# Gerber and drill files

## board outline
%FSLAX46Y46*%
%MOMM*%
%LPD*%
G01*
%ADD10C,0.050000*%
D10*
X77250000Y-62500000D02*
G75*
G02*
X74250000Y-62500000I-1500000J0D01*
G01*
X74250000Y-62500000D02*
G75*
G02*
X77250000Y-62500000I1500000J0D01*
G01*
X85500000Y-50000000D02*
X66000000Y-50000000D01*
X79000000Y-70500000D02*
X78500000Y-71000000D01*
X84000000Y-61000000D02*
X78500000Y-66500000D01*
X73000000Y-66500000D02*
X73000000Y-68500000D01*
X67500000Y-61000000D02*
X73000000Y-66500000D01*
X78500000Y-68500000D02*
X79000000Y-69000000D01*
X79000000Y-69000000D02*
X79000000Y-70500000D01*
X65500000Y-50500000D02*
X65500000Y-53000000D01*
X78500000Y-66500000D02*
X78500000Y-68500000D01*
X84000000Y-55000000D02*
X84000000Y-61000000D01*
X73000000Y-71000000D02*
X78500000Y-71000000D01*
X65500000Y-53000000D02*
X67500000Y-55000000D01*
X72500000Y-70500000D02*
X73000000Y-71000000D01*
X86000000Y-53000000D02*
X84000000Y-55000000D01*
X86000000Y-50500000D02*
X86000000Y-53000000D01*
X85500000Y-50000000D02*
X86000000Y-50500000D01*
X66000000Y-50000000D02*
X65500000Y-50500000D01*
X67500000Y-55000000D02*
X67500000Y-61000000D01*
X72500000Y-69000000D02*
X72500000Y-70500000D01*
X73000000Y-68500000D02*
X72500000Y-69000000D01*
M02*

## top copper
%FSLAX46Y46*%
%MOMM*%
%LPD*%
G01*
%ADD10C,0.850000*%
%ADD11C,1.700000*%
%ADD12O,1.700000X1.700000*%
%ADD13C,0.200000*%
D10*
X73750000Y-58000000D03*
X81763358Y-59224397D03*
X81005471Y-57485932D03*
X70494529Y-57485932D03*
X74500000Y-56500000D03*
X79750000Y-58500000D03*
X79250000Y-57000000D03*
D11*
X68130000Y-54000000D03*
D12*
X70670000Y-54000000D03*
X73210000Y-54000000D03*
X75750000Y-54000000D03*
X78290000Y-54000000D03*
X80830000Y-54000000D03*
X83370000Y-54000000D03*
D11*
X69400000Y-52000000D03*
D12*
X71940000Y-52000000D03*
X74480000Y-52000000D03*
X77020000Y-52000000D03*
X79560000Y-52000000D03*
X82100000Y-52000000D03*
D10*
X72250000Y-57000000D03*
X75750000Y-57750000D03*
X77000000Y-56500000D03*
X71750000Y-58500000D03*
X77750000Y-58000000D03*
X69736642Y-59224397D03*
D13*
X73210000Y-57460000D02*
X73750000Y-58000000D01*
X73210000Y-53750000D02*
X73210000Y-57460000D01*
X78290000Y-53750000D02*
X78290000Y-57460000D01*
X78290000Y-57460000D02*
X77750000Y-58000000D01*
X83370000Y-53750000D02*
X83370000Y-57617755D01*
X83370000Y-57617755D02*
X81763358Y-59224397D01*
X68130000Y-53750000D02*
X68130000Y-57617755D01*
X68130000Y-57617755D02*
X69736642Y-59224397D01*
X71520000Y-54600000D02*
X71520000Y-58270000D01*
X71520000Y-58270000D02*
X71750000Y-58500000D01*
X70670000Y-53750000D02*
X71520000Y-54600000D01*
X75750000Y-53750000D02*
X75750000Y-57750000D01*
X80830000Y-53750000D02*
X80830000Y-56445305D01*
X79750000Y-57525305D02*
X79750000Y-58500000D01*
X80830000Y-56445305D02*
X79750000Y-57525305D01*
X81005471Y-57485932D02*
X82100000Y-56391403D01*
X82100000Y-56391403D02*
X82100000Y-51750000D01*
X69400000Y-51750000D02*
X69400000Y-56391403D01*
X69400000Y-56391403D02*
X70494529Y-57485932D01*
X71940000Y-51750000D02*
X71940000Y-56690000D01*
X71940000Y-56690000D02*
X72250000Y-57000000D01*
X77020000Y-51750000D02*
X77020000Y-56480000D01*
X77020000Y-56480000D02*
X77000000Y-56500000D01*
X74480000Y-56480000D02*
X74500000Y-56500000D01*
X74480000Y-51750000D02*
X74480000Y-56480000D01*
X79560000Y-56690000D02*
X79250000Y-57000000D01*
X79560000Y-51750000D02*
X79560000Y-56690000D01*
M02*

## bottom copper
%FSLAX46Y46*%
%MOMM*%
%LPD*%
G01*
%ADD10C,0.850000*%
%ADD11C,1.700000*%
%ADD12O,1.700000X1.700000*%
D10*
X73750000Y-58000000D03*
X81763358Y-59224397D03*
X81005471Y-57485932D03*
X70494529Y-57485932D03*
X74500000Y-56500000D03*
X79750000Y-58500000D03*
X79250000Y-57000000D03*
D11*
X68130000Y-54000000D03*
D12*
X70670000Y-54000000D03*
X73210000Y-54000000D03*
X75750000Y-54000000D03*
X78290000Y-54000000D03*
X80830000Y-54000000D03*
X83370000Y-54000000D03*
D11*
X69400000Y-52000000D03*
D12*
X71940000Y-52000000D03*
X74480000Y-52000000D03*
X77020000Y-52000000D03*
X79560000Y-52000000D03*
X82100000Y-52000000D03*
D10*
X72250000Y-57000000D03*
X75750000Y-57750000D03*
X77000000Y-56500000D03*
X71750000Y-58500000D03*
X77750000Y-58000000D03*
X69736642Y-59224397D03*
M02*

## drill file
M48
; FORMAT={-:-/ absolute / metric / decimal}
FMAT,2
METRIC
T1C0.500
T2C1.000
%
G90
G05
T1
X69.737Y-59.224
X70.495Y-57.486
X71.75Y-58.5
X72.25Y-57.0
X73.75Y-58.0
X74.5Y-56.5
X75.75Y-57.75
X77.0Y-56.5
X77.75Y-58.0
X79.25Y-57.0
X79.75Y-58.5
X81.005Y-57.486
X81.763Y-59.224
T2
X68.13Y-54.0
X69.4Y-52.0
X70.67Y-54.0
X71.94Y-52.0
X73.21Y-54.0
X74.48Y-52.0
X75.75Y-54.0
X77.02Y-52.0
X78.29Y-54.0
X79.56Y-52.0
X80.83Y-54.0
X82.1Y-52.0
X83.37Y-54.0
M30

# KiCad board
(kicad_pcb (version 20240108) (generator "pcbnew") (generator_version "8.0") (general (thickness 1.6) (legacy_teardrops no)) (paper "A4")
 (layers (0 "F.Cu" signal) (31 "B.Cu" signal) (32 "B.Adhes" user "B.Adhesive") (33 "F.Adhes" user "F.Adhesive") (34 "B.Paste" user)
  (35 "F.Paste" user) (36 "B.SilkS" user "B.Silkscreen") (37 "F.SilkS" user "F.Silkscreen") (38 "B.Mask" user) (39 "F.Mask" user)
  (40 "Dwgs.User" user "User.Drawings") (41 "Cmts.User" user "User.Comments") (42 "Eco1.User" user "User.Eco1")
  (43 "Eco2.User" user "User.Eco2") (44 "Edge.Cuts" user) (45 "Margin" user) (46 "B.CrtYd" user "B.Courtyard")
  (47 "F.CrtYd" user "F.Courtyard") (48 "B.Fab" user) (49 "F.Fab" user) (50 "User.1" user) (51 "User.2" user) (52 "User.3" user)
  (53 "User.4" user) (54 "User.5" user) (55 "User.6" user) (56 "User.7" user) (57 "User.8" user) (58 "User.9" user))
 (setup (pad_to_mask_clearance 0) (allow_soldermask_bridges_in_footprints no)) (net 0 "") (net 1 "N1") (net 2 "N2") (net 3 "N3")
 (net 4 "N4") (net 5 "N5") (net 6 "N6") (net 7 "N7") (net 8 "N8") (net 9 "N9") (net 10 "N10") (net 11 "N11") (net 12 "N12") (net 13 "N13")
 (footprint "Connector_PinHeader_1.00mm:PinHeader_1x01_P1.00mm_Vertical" (layer "F.Cu") (at 73.75 58)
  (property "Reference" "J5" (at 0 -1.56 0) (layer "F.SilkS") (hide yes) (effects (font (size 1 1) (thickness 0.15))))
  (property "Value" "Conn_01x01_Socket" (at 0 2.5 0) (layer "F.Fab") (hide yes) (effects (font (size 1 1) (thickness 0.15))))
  (pad "1" thru_hole circle (at 0 0) (size 0.85 0.85) (drill 0.5) (layers "*.Cu" "*.Mask") (remove_unused_layers no) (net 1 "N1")))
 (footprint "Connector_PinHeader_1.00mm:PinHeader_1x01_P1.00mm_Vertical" (layer "F.Cu") (at 81.763358 59.224397)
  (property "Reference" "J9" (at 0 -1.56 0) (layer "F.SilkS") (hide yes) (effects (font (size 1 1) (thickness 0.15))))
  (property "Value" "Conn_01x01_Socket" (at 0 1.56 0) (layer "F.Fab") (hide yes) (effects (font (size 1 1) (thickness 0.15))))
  (pad "1" thru_hole circle (at 0 0) (size 0.85 0.85) (drill 0.5) (layers "*.Cu" "*.Mask") (remove_unused_layers no) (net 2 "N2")))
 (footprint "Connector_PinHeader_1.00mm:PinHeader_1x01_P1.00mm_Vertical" (layer "F.Cu") (at 81.005471 57.485932)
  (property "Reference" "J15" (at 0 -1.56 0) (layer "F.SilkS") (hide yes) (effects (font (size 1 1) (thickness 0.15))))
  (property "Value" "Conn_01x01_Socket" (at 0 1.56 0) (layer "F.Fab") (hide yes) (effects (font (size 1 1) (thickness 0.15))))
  (pad "1" thru_hole circle (at 0 0) (size 0.85 0.85) (drill 0.5) (layers "*.Cu" "*.Mask") (remove_unused_layers no) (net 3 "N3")))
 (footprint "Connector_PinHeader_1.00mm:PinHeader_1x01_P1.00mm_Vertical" (layer "F.Cu") (at 70.494529 57.485932)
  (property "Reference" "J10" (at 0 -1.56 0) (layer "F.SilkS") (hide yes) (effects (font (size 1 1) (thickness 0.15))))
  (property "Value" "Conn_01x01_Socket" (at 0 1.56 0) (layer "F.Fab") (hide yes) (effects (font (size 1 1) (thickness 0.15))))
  (pad "1" thru_hole circle (at 0 0) (size 0.85 0.85) (drill 0.5) (layers "*.Cu" "*.Mask") (remove_unused_layers no) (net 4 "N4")))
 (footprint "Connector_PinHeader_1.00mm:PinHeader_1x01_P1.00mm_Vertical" (layer "F.Cu") (at 74.5 56.5)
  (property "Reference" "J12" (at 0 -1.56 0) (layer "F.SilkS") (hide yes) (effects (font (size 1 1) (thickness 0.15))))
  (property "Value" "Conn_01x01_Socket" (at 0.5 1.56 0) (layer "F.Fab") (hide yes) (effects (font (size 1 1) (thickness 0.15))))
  (pad "1" thru_hole circle (at 0 0) (size 0.85 0.85) (drill 0.5) (layers "*.Cu" "*.Mask") (remove_unused_layers no) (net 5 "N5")))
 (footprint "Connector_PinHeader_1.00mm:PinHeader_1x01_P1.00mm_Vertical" (layer "F.Cu") (at 79.75 58.5)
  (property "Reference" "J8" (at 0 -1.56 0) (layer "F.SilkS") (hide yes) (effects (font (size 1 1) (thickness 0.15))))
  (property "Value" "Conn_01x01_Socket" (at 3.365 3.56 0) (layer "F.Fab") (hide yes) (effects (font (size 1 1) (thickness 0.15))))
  (pad "1" thru_hole circle (at 0 0) (size 0.85 0.85) (drill 0.5) (layers "*.Cu" "*.Mask") (remove_unused_layers no) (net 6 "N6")))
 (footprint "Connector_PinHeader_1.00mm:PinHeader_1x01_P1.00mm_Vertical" (layer "F.Cu") (at 79.25 57)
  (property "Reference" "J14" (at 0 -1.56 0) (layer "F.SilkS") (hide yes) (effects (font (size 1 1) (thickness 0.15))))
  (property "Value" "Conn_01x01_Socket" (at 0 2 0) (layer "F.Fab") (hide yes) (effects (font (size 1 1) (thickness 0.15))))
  (pad "1" thru_hole circle (at 0 0) (size 0.85 0.85) (drill 0.5) (layers "*.Cu" "*.Mask") (remove_unused_layers no) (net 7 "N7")))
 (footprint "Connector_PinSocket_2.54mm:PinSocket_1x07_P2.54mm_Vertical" (layer "F.Cu") (at 68.13 54 90)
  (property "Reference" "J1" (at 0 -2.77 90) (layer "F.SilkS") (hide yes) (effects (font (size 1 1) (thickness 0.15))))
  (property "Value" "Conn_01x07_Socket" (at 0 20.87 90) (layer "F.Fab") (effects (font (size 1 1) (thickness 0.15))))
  (pad "1" thru_hole circle (at 0 0 90) (size 1.7 1.7) (drill 1) (layers "*.Cu" "*.Mask") (remove_unused_layers no) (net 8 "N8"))
  (pad "2" thru_hole oval (at 0 2.54 90) (size 1.7 1.7) (drill 1) (layers "*.Cu" "*.Mask") (remove_unused_layers no) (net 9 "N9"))
  (pad "3" thru_hole oval (at 0 5.08 90) (size 1.7 1.7) (drill 1) (layers "*.Cu" "*.Mask") (remove_unused_layers no) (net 1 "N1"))
  (pad "4" thru_hole oval (at 0 7.62 90) (size 1.7 1.7) (drill 1) (layers "*.Cu" "*.Mask") (remove_unused_layers no) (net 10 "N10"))
  (pad "5" thru_hole oval (at 0 10.16 90) (size 1.7 1.7) (drill 1) (layers "*.Cu" "*.Mask") (remove_unused_layers no) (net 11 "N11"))
  (pad "6" thru_hole oval (at 0 12.7 90) (size 1.7 1.7) (drill 1) (layers "*.Cu" "*.Mask") (remove_unused_layers no) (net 6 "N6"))
  (pad "7" thru_hole oval (at 0 15.24 90) (size 1.7 1.7) (drill 1) (layers "*.Cu" "*.Mask") (remove_unused_layers no) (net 2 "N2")))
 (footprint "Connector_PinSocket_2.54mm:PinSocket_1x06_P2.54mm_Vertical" (layer "F.Cu") (at 69.4 52 90)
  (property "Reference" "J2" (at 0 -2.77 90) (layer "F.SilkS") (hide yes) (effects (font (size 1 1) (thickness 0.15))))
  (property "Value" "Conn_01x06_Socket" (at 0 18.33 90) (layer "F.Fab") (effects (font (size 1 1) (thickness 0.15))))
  (pad "1" thru_hole circle (at 0 0 90) (size 1.7 1.7) (drill 1) (layers "*.Cu" "*.Mask") (remove_unused_layers no) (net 4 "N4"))
  (pad "2" thru_hole oval (at 0 2.54 90) (size 1.7 1.7) (drill 1) (layers "*.Cu" "*.Mask") (remove_unused_layers no) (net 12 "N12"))
  (pad "3" thru_hole oval (at 0 5.08 90) (size 1.7 1.7) (drill 1) (layers "*.Cu" "*.Mask") (remove_unused_layers no) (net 5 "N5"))
  (pad "4" thru_hole oval (at 0 7.62 90) (size 1.7 1.7) (drill 1) (layers "*.Cu" "*.Mask") (remove_unused_layers no) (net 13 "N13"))
  (pad "5" thru_hole oval (at 0 10.16 90) (size 1.7 1.7) (drill 1) (layers "*.Cu" "*.Mask") (remove_unused_layers no) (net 7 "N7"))
  (pad "6" thru_hole oval (at 0 12.7 90) (size 1.7 1.7) (drill 1) (layers "*.Cu" "*.Mask") (remove_unused_layers no) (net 3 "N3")))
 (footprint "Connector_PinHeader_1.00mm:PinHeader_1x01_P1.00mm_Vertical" (layer "F.Cu") (at 72.25 57)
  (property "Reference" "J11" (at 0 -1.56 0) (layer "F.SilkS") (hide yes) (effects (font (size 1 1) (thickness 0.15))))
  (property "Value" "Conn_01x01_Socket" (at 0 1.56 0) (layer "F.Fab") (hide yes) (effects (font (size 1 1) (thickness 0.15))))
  (pad "1" thru_hole circle (at 0 0) (size 0.85 0.85) (drill 0.5) (layers "*.Cu" "*.Mask") (remove_unused_layers no) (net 12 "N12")))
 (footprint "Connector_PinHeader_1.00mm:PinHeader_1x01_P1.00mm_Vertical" (layer "F.Cu") (at 75.75 57.75)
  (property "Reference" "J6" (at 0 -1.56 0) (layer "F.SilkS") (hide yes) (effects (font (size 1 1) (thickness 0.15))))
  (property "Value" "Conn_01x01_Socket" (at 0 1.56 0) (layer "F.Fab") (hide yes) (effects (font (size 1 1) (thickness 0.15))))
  (pad "1" thru_hole circle (at 0 0) (size 0.85 0.85) (drill 0.5) (layers "*.Cu" "*.Mask") (remove_unused_layers no) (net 10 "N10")))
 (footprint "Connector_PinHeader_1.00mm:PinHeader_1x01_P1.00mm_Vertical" (layer "F.Cu") (at 77 56.5)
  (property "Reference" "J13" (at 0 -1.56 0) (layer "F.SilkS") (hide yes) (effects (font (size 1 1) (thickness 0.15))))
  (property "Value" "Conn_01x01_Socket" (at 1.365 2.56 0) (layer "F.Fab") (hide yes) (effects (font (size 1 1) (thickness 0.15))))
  (pad "1" thru_hole circle (at 0 0) (size 0.85 0.85) (drill 0.5) (layers "*.Cu" "*.Mask") (remove_unused_layers no) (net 13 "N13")))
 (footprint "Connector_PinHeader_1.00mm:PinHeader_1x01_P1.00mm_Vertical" (layer "F.Cu") (at 71.75 58.5)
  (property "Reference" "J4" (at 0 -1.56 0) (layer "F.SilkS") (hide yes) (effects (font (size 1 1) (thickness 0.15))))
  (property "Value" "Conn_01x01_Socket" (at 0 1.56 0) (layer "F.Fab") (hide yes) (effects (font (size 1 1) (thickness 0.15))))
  (pad "1" thru_hole circle (at 0 0) (size 0.85 0.85) (drill 0.5) (layers "*.Cu" "*.Mask") (remove_unused_layers no) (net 9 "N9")))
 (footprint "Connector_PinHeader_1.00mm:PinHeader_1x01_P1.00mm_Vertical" (layer "F.Cu") (at 77.75 58)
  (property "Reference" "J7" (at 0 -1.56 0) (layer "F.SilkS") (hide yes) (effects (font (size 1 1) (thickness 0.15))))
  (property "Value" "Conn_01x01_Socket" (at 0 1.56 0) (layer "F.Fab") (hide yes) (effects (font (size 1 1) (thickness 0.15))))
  (pad "1" thru_hole circle (at 0 0) (size 0.85 0.85) (drill 0.5) (layers "*.Cu" "*.Mask") (remove_unused_layers no) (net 11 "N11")))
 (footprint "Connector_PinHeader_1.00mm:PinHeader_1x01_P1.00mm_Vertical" (layer "F.Cu") (at 69.736642 59.224397)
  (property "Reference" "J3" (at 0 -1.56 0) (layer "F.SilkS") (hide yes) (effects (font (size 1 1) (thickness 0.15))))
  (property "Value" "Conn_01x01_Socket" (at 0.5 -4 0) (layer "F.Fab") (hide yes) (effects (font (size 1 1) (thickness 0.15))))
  (pad "1" thru_hole circle (at 0 0) (size 0.85 0.85) (drill 0.5) (layers "*.Cu" "*.Mask") (remove_unused_layers no) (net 8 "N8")))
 (gr_circle (center 75.75 62.5) (end 75.75 61) (stroke (width 0.05) (type default)) (fill none) (layer "Edge.Cuts"))
 (gr_line (start 85.5 50) (end 66 50) (stroke (width 0.05) (type default)) (layer "Edge.Cuts"))
 (gr_line (start 79 70.5) (end 78.5 71) (stroke (width 0.05) (type default)) (layer "Edge.Cuts"))
 (gr_line (start 84 61) (end 78.5 66.5) (stroke (width 0.05) (type default)) (layer "Edge.Cuts"))
 (gr_line (start 73 66.5) (end 73 68.5) (stroke (width 0.05) (type default)) (layer "Edge.Cuts"))
 (gr_line (start 67.5 61) (end 73 66.5) (stroke (width 0.05) (type default)) (layer "Edge.Cuts"))
 (gr_line (start 78.5 68.5) (end 79 69) (stroke (width 0.05) (type default)) (layer "Edge.Cuts"))
 (gr_line (start 79 69) (end 79 70.5) (stroke (width 0.05) (type default)) (layer "Edge.Cuts"))
 (gr_line (start 65.5 50.5) (end 65.5 53) (stroke (width 0.05) (type default)) (layer "Edge.Cuts"))
 (gr_line (start 78.5 66.5) (end 78.5 68.5) (stroke (width 0.05) (type default)) (layer "Edge.Cuts"))
 (gr_line (start 84 55) (end 84 61) (stroke (width 0.05) (type default)) (layer "Edge.Cuts"))
 (gr_line (start 73 71) (end 78.5 71) (stroke (width 0.05) (type default)) (layer "Edge.Cuts"))
 (gr_line (start 65.5 53) (end 67.5 55) (stroke (width 0.05) (type default)) (layer "Edge.Cuts"))
 (gr_line (start 72.5 70.5) (end 73 71) (stroke (width 0.05) (type default)) (layer "Edge.Cuts"))
 (gr_line (start 86 53) (end 84 55) (stroke (width 0.05) (type default)) (layer "Edge.Cuts"))
 (gr_line (start 86 50.5) (end 86 53) (stroke (width 0.05) (type default)) (layer "Edge.Cuts"))
 (gr_line (start 85.5 50) (end 86 50.5) (stroke (width 0.05) (type default)) (layer "Edge.Cuts"))
 (gr_line (start 66 50) (end 65.5 50.5) (stroke (width 0.05) (type default)) (layer "Edge.Cuts"))
 (gr_line (start 67.5 55) (end 67.5 61) (stroke (width 0.05) (type default)) (layer "Edge.Cuts"))
 (gr_line (start 72.5 69) (end 72.5 70.5) (stroke (width 0.05) (type default)) (layer "Edge.Cuts"))
 (gr_line (start 73 68.5) (end 72.5 69) (stroke (width 0.05) (type default)) (layer "Edge.Cuts"))
 (segment (start 73.21 57.46) (end 73.75 58) (width 0.2) (layer "F.Cu") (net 1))
 (segment (start 73.21 53.75) (end 73.21 57.46) (width 0.2) (layer "F.Cu") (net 1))
 (segment (start 78.29 53.75) (end 78.29 57.46) (width 0.2) (layer "F.Cu") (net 11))
 (segment (start 78.29 57.46) (end 77.75 58) (width 0.2) (layer "F.Cu") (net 11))
 (segment (start 83.37 53.75) (end 83.37 57.617755) (width 0.2) (layer "F.Cu") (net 2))
 (segment (start 83.37 57.617755) (end 81.763358 59.224397) (width 0.2) (layer "F.Cu") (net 2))
 (segment (start 68.13 53.75) (end 68.13 57.617755) (width 0.2) (layer "F.Cu") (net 8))
 (segment (start 68.13 57.617755) (end 69.736642 59.224397) (width 0.2) (layer "F.Cu") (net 8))
 (segment (start 71.52 54.6) (end 71.52 58.27) (width 0.2) (layer "F.Cu") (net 9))
 (segment (start 71.52 58.27) (end 71.75 58.5) (width 0.2) (layer "F.Cu") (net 9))
 (segment (start 70.67 53.75) (end 71.52 54.6) (width 0.2) (layer "F.Cu") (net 9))
 (segment (start 75.75 53.75) (end 75.75 57.75) (width 0.2) (layer "F.Cu") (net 10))
 (segment (start 80.83 53.75) (end 80.83 56.445305) (width 0.2) (layer "F.Cu") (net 6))
 (segment (start 79.75 57.525305) (end 79.75 58.5) (width 0.2) (layer "F.Cu") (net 6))
 (segment (start 80.83 56.445305) (end 79.75 57.525305) (width 0.2) (layer "F.Cu") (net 6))
 (segment (start 81.005471 57.485932) (end 82.1 56.391403) (width 0.2) (layer "F.Cu") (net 3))
 (segment (start 82.1 56.391403) (end 82.1 51.75) (width 0.2) (layer "F.Cu") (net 3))
 (segment (start 69.4 51.75) (end 69.4 56.391403) (width 0.2) (layer "F.Cu") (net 4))
 (segment (start 69.4 56.391403) (end 70.494529 57.485932) (width 0.2) (layer "F.Cu") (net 4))
 (segment (start 71.94 51.75) (end 71.94 56.69) (width 0.2) (layer "F.Cu") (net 12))
 (segment (start 71.94 56.69) (end 72.25 57) (width 0.2) (layer "F.Cu") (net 12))
 (segment (start 77.02 51.75) (end 77.02 56.48) (width 0.2) (layer "F.Cu") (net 13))
 (segment (start 77.02 56.48) (end 77 56.5) (width 0.2) (layer "F.Cu") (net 13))
 (segment (start 74.48 56.48) (end 74.5 56.5) (width 0.2) (layer "F.Cu") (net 5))
 (segment (start 74.48 51.75) (end 74.48 56.48) (width 0.2) (layer "F.Cu") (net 5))
 (segment (start 79.56 56.69) (end 79.25 57) (width 0.2) (layer "F.Cu") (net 7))
 (segment (start 79.56 51.75) (end 79.56 56.69) (width 0.2) (layer "F.Cu") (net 7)))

